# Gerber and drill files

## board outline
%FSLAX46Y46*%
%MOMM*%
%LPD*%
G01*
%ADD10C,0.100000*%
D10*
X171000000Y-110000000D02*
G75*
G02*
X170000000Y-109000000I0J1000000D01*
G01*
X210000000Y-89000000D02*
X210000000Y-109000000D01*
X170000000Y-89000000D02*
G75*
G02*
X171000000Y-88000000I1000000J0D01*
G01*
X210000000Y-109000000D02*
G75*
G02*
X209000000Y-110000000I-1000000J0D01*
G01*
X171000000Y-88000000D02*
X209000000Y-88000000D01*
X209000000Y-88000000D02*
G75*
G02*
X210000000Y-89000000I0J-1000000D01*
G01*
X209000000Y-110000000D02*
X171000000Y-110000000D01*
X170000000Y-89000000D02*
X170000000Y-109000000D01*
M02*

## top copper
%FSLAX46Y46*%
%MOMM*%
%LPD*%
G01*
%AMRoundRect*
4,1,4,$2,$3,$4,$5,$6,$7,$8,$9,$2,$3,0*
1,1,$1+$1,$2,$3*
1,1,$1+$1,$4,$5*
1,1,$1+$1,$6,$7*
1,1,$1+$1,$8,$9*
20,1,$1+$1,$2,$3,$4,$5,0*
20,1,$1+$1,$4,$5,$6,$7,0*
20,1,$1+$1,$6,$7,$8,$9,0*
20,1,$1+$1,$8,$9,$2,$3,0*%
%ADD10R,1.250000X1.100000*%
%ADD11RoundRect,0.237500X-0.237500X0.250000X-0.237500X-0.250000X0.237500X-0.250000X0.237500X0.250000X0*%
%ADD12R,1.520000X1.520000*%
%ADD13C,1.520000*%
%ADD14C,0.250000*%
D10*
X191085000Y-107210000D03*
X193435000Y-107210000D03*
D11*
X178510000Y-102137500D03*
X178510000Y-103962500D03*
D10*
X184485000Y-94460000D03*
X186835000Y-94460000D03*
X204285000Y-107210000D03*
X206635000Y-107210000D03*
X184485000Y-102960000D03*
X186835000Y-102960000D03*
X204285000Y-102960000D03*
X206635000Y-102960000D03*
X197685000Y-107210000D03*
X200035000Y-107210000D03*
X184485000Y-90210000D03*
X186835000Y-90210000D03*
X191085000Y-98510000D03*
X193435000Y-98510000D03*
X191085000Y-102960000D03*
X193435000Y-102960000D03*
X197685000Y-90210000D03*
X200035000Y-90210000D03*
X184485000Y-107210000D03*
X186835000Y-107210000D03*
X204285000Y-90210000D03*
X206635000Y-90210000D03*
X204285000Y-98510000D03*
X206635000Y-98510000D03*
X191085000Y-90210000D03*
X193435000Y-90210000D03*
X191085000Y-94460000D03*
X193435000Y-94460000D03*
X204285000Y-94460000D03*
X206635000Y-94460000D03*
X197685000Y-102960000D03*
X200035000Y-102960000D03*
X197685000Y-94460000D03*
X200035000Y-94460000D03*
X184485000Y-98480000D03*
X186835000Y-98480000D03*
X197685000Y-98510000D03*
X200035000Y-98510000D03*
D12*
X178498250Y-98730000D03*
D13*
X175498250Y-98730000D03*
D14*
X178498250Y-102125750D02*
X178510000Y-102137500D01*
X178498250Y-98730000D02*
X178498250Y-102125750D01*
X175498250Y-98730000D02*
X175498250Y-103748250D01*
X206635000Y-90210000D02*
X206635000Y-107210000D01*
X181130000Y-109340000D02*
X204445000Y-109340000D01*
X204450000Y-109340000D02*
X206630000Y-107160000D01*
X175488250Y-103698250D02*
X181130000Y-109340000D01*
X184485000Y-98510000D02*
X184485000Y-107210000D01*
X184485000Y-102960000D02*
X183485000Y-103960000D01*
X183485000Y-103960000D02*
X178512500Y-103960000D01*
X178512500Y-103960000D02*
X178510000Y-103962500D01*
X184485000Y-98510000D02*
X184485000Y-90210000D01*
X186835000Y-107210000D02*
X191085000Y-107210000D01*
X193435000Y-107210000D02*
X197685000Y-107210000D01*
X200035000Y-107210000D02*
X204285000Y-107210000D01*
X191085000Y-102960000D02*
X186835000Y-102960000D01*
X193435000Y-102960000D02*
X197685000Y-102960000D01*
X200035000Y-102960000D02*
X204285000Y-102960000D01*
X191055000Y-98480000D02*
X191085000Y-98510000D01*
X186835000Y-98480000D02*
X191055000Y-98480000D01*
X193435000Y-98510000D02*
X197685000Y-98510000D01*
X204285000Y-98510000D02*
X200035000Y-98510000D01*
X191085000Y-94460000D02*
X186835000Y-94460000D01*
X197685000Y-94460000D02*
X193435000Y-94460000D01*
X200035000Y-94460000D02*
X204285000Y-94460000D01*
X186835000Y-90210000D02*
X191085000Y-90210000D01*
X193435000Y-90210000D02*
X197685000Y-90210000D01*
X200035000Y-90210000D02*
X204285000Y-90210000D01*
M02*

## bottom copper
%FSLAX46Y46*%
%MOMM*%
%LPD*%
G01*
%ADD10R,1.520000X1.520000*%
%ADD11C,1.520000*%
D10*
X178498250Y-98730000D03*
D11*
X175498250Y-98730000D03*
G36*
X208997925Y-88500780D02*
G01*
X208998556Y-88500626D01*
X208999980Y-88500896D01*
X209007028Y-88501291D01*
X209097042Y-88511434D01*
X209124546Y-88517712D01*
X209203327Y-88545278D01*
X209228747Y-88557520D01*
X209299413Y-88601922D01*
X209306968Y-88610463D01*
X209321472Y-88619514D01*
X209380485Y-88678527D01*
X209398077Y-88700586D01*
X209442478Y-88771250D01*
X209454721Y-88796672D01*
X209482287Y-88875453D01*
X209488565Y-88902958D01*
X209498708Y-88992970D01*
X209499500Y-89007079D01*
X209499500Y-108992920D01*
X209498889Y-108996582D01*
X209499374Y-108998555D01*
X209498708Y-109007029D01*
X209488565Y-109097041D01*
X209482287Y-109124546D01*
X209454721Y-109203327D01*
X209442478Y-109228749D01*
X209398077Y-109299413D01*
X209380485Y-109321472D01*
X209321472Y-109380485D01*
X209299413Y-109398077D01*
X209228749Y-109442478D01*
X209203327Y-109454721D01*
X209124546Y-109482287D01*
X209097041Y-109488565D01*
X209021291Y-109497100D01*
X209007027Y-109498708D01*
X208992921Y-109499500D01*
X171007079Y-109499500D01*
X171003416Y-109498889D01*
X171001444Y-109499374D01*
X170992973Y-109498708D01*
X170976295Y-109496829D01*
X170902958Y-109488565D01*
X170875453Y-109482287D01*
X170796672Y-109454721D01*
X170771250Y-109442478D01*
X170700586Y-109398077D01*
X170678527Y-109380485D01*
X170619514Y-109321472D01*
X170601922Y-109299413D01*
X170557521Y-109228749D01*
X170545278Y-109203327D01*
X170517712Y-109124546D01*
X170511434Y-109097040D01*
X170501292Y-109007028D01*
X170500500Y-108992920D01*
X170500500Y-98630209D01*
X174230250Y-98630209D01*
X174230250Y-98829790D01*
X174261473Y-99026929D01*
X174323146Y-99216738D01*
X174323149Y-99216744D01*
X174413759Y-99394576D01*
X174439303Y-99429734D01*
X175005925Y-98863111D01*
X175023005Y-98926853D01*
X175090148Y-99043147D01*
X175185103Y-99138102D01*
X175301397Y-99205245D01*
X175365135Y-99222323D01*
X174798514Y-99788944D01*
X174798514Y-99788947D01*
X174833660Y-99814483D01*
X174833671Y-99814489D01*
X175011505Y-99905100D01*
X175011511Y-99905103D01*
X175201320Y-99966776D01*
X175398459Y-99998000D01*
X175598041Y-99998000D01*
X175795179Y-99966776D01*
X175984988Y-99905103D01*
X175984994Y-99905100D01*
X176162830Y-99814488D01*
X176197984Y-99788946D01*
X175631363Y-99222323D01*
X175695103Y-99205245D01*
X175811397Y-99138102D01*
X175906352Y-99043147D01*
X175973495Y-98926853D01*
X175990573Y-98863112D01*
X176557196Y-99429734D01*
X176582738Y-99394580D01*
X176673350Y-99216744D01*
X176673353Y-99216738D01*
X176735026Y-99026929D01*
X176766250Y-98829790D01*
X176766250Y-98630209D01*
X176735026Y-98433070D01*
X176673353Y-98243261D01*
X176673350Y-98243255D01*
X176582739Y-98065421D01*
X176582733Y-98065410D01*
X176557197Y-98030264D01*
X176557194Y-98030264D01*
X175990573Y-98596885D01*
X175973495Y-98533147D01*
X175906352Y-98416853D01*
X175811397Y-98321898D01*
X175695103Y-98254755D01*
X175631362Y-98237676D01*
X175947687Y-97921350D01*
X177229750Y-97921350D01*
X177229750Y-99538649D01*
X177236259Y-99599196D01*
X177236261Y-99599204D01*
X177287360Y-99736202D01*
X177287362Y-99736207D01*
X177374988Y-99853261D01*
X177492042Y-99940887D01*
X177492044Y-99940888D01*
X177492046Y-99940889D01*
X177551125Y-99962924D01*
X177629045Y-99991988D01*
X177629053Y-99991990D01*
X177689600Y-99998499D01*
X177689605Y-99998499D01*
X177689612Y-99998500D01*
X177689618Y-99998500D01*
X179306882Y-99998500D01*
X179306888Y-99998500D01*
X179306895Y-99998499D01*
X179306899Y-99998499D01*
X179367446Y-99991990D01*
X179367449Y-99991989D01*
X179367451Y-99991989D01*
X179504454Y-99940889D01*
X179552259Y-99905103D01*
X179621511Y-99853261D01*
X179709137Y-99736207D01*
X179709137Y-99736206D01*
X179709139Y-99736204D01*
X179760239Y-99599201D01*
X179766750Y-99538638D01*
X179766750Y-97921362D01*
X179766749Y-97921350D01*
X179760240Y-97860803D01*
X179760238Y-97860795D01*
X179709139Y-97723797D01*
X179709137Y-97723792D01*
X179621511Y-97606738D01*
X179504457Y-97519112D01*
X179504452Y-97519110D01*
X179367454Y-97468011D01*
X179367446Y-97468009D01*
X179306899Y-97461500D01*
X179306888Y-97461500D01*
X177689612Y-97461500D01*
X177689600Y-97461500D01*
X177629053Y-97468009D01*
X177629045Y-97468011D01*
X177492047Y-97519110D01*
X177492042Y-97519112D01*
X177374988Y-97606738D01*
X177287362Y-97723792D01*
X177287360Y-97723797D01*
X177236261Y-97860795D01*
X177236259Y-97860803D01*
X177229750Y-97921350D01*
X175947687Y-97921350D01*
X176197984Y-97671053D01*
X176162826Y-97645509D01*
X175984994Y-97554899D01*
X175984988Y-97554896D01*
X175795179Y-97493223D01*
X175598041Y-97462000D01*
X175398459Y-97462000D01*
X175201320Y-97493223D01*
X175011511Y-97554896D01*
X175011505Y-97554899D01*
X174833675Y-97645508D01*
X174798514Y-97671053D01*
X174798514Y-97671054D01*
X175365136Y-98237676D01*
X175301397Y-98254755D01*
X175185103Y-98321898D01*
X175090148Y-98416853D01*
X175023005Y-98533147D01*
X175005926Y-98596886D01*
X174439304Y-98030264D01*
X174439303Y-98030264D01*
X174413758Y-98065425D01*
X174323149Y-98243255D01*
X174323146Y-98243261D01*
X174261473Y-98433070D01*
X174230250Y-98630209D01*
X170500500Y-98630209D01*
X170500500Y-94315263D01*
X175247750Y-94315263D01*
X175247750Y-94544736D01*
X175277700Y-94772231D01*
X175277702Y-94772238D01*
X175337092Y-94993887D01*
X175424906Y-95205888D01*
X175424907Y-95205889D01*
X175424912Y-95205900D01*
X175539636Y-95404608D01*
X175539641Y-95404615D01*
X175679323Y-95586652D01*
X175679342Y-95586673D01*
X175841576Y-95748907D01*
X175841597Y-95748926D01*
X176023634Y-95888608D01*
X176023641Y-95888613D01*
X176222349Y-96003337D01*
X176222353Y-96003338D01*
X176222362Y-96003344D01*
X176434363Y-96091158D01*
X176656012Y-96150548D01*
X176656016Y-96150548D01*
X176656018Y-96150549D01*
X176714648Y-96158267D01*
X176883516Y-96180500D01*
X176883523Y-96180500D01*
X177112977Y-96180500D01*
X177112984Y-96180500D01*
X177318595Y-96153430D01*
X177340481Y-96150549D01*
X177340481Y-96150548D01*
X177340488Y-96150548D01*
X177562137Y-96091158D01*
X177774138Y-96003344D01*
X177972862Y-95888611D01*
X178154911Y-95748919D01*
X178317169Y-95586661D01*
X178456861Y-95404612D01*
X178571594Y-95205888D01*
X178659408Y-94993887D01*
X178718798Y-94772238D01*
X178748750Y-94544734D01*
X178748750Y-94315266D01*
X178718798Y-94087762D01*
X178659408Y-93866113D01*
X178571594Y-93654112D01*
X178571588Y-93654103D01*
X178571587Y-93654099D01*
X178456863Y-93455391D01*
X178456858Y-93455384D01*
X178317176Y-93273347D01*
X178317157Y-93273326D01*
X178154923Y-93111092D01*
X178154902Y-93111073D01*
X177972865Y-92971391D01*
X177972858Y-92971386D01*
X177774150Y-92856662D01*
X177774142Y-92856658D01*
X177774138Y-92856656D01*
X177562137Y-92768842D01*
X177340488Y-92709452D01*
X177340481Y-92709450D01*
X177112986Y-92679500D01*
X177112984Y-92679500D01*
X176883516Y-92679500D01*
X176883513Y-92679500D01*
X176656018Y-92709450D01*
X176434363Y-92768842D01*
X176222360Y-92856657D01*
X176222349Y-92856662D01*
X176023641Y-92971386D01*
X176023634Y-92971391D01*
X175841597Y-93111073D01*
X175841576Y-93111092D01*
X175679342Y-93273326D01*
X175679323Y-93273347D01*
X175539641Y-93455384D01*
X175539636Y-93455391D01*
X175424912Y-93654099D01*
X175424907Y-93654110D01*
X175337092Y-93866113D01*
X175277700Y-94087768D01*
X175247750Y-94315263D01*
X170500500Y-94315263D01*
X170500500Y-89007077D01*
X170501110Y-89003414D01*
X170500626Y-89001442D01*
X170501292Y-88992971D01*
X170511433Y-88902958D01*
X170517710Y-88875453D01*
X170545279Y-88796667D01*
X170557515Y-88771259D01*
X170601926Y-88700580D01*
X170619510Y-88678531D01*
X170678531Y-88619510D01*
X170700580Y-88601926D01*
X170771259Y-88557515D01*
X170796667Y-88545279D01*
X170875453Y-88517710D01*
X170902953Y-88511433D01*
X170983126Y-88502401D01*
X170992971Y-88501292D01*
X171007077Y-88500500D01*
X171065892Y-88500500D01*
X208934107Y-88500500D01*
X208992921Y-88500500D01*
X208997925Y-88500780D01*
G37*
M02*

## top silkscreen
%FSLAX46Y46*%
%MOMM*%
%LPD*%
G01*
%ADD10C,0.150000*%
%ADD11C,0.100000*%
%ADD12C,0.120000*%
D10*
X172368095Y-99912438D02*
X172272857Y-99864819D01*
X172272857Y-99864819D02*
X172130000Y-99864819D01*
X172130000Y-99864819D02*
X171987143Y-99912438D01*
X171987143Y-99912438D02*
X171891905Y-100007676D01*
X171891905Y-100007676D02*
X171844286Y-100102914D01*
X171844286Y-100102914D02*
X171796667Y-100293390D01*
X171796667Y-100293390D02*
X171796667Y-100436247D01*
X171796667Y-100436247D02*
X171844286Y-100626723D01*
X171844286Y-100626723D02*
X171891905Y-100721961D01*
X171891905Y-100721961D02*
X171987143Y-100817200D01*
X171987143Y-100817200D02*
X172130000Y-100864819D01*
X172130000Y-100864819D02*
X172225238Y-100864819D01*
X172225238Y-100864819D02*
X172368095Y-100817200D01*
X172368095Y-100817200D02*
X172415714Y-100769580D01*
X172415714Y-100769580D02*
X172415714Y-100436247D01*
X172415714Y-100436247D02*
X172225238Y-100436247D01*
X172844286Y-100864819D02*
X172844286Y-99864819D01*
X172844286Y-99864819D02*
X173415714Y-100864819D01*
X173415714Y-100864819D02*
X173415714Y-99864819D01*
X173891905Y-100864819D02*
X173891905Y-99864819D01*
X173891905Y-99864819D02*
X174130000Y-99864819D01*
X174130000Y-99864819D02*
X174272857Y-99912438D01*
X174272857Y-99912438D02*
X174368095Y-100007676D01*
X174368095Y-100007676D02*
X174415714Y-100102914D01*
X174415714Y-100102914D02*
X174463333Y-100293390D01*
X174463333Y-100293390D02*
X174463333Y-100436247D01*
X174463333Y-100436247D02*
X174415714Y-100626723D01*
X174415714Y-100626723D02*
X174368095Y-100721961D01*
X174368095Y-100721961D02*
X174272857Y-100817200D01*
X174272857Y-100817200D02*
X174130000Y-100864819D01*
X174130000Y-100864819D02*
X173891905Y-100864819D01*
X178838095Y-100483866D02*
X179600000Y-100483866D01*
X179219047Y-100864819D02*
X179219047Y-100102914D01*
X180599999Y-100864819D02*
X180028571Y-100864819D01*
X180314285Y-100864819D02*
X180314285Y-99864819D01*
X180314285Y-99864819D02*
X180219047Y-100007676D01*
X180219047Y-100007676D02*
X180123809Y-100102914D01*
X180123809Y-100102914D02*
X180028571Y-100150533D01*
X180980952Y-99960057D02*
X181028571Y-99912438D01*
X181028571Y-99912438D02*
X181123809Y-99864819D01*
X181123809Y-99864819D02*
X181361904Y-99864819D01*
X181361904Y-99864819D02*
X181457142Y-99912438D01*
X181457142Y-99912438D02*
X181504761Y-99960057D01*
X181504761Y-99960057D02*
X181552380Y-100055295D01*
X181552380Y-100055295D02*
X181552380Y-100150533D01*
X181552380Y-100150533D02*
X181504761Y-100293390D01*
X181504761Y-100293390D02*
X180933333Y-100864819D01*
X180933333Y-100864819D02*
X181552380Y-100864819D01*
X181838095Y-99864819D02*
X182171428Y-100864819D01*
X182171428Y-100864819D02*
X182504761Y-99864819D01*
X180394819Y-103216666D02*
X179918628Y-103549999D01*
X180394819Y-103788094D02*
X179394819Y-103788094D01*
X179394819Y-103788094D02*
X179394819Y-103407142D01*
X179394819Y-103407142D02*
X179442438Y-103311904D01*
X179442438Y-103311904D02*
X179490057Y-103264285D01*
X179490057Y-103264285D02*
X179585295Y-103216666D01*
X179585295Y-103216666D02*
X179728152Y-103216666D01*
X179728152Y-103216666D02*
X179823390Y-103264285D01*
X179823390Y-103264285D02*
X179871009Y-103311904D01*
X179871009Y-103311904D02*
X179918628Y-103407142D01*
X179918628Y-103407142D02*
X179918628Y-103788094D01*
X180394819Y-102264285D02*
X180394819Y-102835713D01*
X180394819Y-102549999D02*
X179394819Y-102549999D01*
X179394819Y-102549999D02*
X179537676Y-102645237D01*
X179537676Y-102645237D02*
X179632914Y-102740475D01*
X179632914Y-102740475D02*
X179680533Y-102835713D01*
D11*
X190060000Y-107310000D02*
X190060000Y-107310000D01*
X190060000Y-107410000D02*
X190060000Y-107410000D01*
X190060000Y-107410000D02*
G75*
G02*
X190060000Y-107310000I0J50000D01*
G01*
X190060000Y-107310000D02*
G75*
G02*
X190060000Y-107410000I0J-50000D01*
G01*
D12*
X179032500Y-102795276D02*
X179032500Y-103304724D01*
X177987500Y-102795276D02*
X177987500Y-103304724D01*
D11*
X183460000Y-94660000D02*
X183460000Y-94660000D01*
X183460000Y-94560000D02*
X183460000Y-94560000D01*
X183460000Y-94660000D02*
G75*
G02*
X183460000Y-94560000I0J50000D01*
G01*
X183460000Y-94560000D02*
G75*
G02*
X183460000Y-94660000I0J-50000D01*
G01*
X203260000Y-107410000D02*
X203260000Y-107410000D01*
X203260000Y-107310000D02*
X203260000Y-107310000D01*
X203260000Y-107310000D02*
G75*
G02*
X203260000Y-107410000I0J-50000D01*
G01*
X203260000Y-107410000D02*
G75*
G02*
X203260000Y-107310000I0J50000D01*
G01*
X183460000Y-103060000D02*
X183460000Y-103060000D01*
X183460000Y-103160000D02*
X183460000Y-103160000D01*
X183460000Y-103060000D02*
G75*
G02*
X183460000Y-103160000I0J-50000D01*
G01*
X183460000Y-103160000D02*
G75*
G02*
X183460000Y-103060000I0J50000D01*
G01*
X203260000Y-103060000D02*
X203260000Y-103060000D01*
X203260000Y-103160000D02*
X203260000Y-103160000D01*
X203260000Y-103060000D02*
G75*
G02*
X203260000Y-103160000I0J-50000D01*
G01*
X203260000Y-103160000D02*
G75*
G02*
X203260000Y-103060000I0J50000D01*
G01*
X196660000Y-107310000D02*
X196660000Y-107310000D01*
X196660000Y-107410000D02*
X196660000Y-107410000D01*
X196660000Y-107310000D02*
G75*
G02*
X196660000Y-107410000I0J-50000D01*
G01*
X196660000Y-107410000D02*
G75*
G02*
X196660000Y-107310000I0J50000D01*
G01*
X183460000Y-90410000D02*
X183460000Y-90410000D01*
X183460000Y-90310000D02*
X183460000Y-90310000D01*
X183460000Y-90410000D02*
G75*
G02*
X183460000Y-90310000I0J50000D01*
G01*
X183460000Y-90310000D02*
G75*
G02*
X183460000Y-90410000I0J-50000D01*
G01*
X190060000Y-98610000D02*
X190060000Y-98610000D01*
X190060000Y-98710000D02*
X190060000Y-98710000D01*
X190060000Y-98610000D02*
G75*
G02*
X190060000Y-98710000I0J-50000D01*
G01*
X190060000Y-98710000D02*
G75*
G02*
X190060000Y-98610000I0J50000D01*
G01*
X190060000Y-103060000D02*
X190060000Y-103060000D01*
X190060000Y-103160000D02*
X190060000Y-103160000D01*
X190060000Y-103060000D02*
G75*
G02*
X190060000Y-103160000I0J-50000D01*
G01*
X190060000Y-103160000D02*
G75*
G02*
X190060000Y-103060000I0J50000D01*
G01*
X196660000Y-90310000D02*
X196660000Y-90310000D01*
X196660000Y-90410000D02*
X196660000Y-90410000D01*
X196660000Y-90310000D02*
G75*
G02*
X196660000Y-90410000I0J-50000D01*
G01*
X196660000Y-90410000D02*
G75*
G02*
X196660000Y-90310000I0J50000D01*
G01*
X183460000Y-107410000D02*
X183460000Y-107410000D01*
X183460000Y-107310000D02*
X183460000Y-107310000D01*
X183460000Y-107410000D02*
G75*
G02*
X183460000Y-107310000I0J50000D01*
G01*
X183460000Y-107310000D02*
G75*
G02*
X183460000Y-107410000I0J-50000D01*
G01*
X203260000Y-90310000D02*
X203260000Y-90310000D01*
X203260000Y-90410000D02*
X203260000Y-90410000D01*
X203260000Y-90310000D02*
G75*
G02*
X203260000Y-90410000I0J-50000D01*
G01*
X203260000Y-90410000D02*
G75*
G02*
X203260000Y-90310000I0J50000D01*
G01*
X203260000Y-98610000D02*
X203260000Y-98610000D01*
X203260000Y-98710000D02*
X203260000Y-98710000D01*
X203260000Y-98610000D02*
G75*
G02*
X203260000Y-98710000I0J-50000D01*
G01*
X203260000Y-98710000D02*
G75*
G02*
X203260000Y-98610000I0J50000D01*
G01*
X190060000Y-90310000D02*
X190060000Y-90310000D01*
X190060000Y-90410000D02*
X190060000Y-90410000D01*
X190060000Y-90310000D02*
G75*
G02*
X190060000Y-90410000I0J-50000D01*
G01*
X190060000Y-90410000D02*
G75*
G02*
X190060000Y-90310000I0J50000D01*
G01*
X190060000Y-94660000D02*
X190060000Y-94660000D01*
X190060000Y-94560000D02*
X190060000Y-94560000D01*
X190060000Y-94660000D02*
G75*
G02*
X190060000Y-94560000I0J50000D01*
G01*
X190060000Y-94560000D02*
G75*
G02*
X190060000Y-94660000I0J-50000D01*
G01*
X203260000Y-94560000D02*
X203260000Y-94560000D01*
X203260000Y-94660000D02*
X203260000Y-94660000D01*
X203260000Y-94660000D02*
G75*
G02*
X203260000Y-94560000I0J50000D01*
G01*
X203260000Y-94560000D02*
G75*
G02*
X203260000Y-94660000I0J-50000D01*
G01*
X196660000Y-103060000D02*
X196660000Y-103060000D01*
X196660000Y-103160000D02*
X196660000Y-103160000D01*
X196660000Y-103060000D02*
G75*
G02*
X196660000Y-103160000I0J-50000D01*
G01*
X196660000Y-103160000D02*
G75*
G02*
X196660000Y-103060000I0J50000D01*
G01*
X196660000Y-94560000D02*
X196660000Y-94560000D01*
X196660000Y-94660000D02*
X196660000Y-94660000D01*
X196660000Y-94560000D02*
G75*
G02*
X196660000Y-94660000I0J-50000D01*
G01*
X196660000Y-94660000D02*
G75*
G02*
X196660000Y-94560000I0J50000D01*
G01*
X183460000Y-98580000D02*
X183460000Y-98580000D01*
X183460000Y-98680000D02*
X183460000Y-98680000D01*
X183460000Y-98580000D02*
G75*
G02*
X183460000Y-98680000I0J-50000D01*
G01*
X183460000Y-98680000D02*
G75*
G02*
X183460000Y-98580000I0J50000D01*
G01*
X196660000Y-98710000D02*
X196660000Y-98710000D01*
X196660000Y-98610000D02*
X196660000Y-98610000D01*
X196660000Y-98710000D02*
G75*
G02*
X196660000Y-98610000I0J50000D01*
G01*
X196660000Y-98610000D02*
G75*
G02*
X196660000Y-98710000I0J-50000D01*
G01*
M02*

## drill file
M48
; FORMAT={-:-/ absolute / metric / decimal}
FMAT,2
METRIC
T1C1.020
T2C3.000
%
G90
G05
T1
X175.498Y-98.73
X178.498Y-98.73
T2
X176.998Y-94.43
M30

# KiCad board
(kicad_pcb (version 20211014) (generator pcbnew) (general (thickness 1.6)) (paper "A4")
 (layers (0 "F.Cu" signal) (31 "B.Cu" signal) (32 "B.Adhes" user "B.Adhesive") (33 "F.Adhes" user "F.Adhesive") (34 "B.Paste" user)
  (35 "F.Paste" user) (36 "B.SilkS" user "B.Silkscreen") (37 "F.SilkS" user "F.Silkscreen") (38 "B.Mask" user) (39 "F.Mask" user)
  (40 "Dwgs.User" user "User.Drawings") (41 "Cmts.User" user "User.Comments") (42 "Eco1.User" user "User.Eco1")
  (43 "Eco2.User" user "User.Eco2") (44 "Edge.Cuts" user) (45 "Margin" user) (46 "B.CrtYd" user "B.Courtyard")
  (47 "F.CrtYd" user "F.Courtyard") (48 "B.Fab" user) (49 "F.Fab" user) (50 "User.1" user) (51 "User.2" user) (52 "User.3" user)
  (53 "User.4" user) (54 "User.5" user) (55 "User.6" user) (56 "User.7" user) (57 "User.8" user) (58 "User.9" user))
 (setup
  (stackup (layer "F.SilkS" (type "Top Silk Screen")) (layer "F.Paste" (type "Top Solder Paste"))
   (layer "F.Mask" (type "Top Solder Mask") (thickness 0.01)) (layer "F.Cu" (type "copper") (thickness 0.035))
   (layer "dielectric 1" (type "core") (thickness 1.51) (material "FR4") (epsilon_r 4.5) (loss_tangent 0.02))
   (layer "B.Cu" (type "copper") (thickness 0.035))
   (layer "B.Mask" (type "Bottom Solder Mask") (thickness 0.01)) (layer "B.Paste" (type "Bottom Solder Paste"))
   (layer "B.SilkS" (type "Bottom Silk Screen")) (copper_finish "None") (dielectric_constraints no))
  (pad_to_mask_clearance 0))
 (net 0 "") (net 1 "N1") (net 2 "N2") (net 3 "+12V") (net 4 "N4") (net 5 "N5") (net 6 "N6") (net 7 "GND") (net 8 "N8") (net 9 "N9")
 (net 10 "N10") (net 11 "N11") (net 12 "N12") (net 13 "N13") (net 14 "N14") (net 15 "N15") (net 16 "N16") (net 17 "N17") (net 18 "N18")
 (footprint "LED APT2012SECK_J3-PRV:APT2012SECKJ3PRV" (layer "F.Cu") (at 192.26 107.21)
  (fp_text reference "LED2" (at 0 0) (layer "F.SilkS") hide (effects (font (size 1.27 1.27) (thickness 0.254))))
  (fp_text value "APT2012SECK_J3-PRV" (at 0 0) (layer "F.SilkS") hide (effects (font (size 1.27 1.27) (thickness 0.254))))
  (fp_line (start -2.2 0.1) (end -2.2 0.1) (layer "F.SilkS") (width 0.1))
  (fp_line (start -2.2 0.2) (end -2.2 0.2) (layer "F.SilkS") (width 0.1))
  (fp_arc (start -2.2 0.2) (mid -2.25 0.15) (end -2.2 0.1) (layer "F.SilkS") (width 0.1))
  (fp_arc (start -2.2 0.1) (mid -2.15 0.15) (end -2.2 0.2) (layer "F.SilkS") (width 0.1))
  (pad "1" smd rect (at -1.175 0 90) (size 1.1 1.25) (layers "F.Cu" "F.Paste" "F.Mask") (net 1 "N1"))
  (pad "2" smd rect (at 1.175 0 90) (size 1.1 1.25) (layers "F.Cu" "F.Paste" "F.Mask") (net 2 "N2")))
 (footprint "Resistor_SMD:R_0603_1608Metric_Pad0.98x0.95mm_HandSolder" (layer "F.Cu") (at 178.51 103.05 -90)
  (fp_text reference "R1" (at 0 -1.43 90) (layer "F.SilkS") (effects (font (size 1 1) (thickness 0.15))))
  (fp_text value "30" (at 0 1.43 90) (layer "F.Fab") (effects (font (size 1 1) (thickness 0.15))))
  (fp_line (start -0.254724 -0.5225) (end 0.254724 -0.5225) (layer "F.SilkS") (width 0.12))
  (fp_line (start -0.254724 0.5225) (end 0.254724 0.5225) (layer "F.SilkS") (width 0.12))
  (pad "1" smd roundrect locked (at -0.9125 0 270) (size 0.975 0.95) (layers "F.Cu" "F.Paste" "F.Mask") (roundrect_rratio 0.25)
   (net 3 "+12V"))
  (pad "2" smd roundrect locked (at 0.9125 0 270) (size 0.975 0.95) (layers "F.Cu" "F.Paste" "F.Mask") (roundrect_rratio 0.25) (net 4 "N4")))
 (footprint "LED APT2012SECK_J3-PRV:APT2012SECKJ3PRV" (layer "F.Cu") (at 185.66 94.46)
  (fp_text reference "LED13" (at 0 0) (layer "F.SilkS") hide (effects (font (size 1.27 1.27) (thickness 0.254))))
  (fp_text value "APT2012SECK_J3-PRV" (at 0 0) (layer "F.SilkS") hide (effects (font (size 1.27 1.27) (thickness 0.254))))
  (fp_line (start -2.2 0.2) (end -2.2 0.2) (layer "F.SilkS") (width 0.1))
  (fp_line (start -2.2 0.1) (end -2.2 0.1) (layer "F.SilkS") (width 0.1))
  (fp_arc (start -2.2 0.2) (mid -2.25 0.15) (end -2.2 0.1) (layer "F.SilkS") (width 0.1))
  (fp_arc (start -2.2 0.1) (mid -2.15 0.15) (end -2.2 0.2) (layer "F.SilkS") (width 0.1))
  (pad "1" smd rect (at -1.175 0 90) (size 1.1 1.25) (layers "F.Cu" "F.Paste" "F.Mask") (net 4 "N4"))
  (pad "2" smd rect (at 1.175 0 90) (size 1.1 1.25) (layers "F.Cu" "F.Paste" "F.Mask") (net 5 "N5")))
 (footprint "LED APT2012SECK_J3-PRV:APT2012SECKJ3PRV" (layer "F.Cu") (at 205.46 107.21)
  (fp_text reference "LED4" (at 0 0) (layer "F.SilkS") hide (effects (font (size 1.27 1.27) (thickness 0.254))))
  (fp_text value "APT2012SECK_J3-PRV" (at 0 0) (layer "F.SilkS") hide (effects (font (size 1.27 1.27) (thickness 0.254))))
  (fp_line (start -2.2 0.2) (end -2.2 0.2) (layer "F.SilkS") (width 0.1))
  (fp_line (start -2.2 0.1) (end -2.2 0.1) (layer "F.SilkS") (width 0.1))
  (fp_arc (start -2.2 0.1) (mid -2.15 0.15) (end -2.2 0.2) (layer "F.SilkS") (width 0.1))
  (fp_arc (start -2.2 0.2) (mid -2.25 0.15) (end -2.2 0.1) (layer "F.SilkS") (width 0.1))
  (pad "1" smd rect (at -1.175 0 90) (size 1.1 1.25) (layers "F.Cu" "F.Paste" "F.Mask") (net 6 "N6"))
  (pad "2" smd rect (at 1.175 0 90) (size 1.1 1.25) (layers "F.Cu" "F.Paste" "F.Mask") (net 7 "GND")))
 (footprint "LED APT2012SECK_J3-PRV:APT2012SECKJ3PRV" (layer "F.Cu") (at 185.66 102.96)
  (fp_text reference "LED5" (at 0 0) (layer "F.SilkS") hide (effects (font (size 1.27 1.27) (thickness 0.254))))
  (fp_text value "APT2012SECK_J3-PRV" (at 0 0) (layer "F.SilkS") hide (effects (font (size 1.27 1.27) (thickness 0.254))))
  (fp_line (start -2.2 0.1) (end -2.2 0.1) (layer "F.SilkS") (width 0.1))
  (fp_line (start -2.2 0.2) (end -2.2 0.2) (layer "F.SilkS") (width 0.1))
  (fp_arc (start -2.2 0.1) (mid -2.15 0.15) (end -2.2 0.2) (layer "F.SilkS") (width 0.1))
  (fp_arc (start -2.2 0.2) (mid -2.25 0.15) (end -2.2 0.1) (layer "F.SilkS") (width 0.1))
  (pad "1" smd rect (at -1.175 0 90) (size 1.1 1.25) (layers "F.Cu" "F.Paste" "F.Mask") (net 4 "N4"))
  (pad "2" smd rect (at 1.175 0 90) (size 1.1 1.25) (layers "F.Cu" "F.Paste" "F.Mask") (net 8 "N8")))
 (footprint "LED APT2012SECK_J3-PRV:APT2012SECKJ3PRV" (layer "F.Cu") (at 205.46 102.96)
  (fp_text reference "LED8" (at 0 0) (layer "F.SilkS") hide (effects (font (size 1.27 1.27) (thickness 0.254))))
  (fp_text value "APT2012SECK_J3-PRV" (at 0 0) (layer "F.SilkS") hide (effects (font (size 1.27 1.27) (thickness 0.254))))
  (fp_line (start -2.2 0.1) (end -2.2 0.1) (layer "F.SilkS") (width 0.1))
  (fp_line (start -2.2 0.2) (end -2.2 0.2) (layer "F.SilkS") (width 0.1))
  (fp_arc (start -2.2 0.1) (mid -2.15 0.15) (end -2.2 0.2) (layer "F.SilkS") (width 0.1))
  (fp_arc (start -2.2 0.2) (mid -2.25 0.15) (end -2.2 0.1) (layer "F.SilkS") (width 0.1))
  (pad "1" smd rect (at -1.175 0 90) (size 1.1 1.25) (layers "F.Cu" "F.Paste" "F.Mask") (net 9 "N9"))
  (pad "2" smd rect (at 1.175 0 90) (size 1.1 1.25) (layers "F.Cu" "F.Paste" "F.Mask") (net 7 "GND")))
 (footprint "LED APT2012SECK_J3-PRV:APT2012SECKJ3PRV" (layer "F.Cu") (at 198.86 107.21)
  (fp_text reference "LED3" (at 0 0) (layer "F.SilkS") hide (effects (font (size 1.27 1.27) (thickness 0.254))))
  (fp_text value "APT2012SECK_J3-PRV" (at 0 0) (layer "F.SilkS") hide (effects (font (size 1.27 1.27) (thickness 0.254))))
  (fp_line (start -2.2 0.1) (end -2.2 0.1) (layer "F.SilkS") (width 0.1))
  (fp_line (start -2.2 0.2) (end -2.2 0.2) (layer "F.SilkS") (width 0.1))
  (fp_arc (start -2.2 0.1) (mid -2.15 0.15) (end -2.2 0.2) (layer "F.SilkS") (width 0.1))
  (fp_arc (start -2.2 0.2) (mid -2.25 0.15) (end -2.2 0.1) (layer "F.SilkS") (width 0.1))
  (pad "1" smd rect (at -1.175 0 90) (size 1.1 1.25) (layers "F.Cu" "F.Paste" "F.Mask") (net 2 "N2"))
  (pad "2" smd rect (at 1.175 0 90) (size 1.1 1.25) (layers "F.Cu" "F.Paste" "F.Mask") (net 6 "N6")))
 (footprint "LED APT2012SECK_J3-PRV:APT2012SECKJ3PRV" (layer "F.Cu") (at 185.66 90.21)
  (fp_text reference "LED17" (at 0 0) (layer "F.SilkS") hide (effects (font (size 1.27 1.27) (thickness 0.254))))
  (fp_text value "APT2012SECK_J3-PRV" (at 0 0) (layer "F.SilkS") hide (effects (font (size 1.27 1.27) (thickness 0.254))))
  (fp_line (start -2.2 0.2) (end -2.2 0.2) (layer "F.SilkS") (width 0.1))
  (fp_line (start -2.2 0.1) (end -2.2 0.1) (layer "F.SilkS") (width 0.1))
  (fp_arc (start -2.2 0.2) (mid -2.25 0.15) (end -2.2 0.1) (layer "F.SilkS") (width 0.1))
  (fp_arc (start -2.2 0.1) (mid -2.15 0.15) (end -2.2 0.2) (layer "F.SilkS") (width 0.1))
  (pad "1" smd rect (at -1.175 0 90) (size 1.1 1.25) (layers "F.Cu" "F.Paste" "F.Mask") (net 4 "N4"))
  (pad "2" smd rect (at 1.175 0 90) (size 1.1 1.25) (layers "F.Cu" "F.Paste" "F.Mask") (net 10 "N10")))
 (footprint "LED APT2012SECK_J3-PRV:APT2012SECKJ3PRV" (layer "F.Cu") (at 192.26 98.51)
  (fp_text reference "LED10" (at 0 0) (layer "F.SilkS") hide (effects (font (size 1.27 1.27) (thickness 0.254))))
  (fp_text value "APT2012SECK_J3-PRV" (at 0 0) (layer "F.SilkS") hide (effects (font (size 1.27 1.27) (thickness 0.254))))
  (fp_line (start -2.2 0.1) (end -2.2 0.1) (layer "F.SilkS") (width 0.1))
  (fp_line (start -2.2 0.2) (end -2.2 0.2) (layer "F.SilkS") (width 0.1))
  (fp_arc (start -2.2 0.1) (mid -2.15 0.15) (end -2.2 0.2) (layer "F.SilkS") (width 0.1))
  (fp_arc (start -2.2 0.2) (mid -2.25 0.15) (end -2.2 0.1) (layer "F.SilkS") (width 0.1))
  (pad "1" smd rect (at -1.175 0 90) (size 1.1 1.25) (layers "F.Cu" "F.Paste" "F.Mask") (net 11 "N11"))
  (pad "2" smd rect (at 1.175 0 90) (size 1.1 1.25) (layers "F.Cu" "F.Paste" "F.Mask") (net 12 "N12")))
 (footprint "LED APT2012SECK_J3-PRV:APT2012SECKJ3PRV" (layer "F.Cu") (at 192.26 102.96)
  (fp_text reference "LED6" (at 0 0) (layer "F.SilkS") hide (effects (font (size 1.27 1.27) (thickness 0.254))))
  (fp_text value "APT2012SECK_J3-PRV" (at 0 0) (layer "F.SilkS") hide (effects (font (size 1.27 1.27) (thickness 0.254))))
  (fp_line (start -2.2 0.1) (end -2.2 0.1) (layer "F.SilkS") (width 0.1))
  (fp_line (start -2.2 0.2) (end -2.2 0.2) (layer "F.SilkS") (width 0.1))
  (fp_arc (start -2.2 0.1) (mid -2.15 0.15) (end -2.2 0.2) (layer "F.SilkS") (width 0.1))
  (fp_arc (start -2.2 0.2) (mid -2.25 0.15) (end -2.2 0.1) (layer "F.SilkS") (width 0.1))
  (pad "1" smd rect (at -1.175 0 90) (size 1.1 1.25) (layers "F.Cu" "F.Paste" "F.Mask") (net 8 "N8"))
  (pad "2" smd rect (at 1.175 0 90) (size 1.1 1.25) (layers "F.Cu" "F.Paste" "F.Mask") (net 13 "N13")))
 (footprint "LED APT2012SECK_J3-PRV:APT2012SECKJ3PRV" (layer "F.Cu") (at 198.86 90.21)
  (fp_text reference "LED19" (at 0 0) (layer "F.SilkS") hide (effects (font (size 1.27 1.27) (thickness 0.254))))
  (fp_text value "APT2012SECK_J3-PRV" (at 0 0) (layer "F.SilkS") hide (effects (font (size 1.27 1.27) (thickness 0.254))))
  (fp_line (start -2.2 0.1) (end -2.2 0.1) (layer "F.SilkS") (width 0.1))
  (fp_line (start -2.2 0.2) (end -2.2 0.2) (layer "F.SilkS") (width 0.1))
  (fp_arc (start -2.2 0.1) (mid -2.15 0.15) (end -2.2 0.2) (layer "F.SilkS") (width 0.1))
  (fp_arc (start -2.2 0.2) (mid -2.25 0.15) (end -2.2 0.1) (layer "F.SilkS") (width 0.1))
  (pad "1" smd rect (at -1.175 0 90) (size 1.1 1.25) (layers "F.Cu" "F.Paste" "F.Mask") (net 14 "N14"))
  (pad "2" smd rect (at 1.175 0 90) (size 1.1 1.25) (layers "F.Cu" "F.Paste" "F.Mask") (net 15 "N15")))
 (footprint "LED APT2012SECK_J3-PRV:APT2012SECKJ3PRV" (layer "F.Cu") (at 185.66 107.21)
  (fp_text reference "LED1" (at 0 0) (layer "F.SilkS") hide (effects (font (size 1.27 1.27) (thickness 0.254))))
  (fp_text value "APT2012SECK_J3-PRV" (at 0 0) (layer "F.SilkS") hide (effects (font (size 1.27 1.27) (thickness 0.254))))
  (fp_line (start -2.2 0.2) (end -2.2 0.2) (layer "F.SilkS") (width 0.1))
  (fp_line (start -2.2 0.1) (end -2.2 0.1) (layer "F.SilkS") (width 0.1))
  (fp_arc (start -2.2 0.2) (mid -2.25 0.15) (end -2.2 0.1) (layer "F.SilkS") (width 0.1))
  (fp_arc (start -2.2 0.1) (mid -2.15 0.15) (end -2.2 0.2) (layer "F.SilkS") (width 0.1))
  (pad "1" smd rect (at -1.175 0 90) (size 1.1 1.25) (layers "F.Cu" "F.Paste" "F.Mask") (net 4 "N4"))
  (pad "2" smd rect (at 1.175 0 90) (size 1.1 1.25) (layers "F.Cu" "F.Paste" "F.Mask") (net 1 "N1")))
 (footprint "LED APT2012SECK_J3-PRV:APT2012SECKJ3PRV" (layer "F.Cu") (at 205.46 90.21)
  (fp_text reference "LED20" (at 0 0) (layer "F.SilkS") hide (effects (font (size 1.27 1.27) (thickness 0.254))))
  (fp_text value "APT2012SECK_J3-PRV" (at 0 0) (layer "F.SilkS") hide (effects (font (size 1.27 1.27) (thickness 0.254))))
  (fp_line (start -2.2 0.1) (end -2.2 0.1) (layer "F.SilkS") (width 0.1))
  (fp_line (start -2.2 0.2) (end -2.2 0.2) (layer "F.SilkS") (width 0.1))
  (fp_arc (start -2.2 0.1) (mid -2.15 0.15) (end -2.2 0.2) (layer "F.SilkS") (width 0.1))
  (fp_arc (start -2.2 0.2) (mid -2.25 0.15) (end -2.2 0.1) (layer "F.SilkS") (width 0.1))
  (pad "1" smd rect (at -1.175 0 90) (size 1.1 1.25) (layers "F.Cu" "F.Paste" "F.Mask") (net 15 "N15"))
  (pad "2" smd rect (at 1.175 0 90) (size 1.1 1.25) (layers "F.Cu" "F.Paste" "F.Mask") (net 7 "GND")))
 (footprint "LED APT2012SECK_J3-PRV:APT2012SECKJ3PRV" (layer "F.Cu") (at 205.46 98.51)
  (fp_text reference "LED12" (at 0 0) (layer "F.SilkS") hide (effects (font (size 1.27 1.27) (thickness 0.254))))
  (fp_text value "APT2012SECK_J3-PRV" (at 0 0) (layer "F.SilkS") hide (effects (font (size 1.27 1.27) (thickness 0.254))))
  (fp_line (start -2.2 0.1) (end -2.2 0.1) (layer "F.SilkS") (width 0.1))
  (fp_line (start -2.2 0.2) (end -2.2 0.2) (layer "F.SilkS") (width 0.1))
  (fp_arc (start -2.2 0.1) (mid -2.15 0.15) (end -2.2 0.2) (layer "F.SilkS") (width 0.1))
  (fp_arc (start -2.2 0.2) (mid -2.25 0.15) (end -2.2 0.1) (layer "F.SilkS") (width 0.1))
  (pad "1" smd rect (at -1.175 0 90) (size 1.1 1.25) (layers "F.Cu" "F.Paste" "F.Mask") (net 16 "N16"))
  (pad "2" smd rect (at 1.175 0 90) (size 1.1 1.25) (layers "F.Cu" "F.Paste" "F.Mask") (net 7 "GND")))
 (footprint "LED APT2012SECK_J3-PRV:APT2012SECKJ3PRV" (layer "F.Cu") (at 192.26 90.21)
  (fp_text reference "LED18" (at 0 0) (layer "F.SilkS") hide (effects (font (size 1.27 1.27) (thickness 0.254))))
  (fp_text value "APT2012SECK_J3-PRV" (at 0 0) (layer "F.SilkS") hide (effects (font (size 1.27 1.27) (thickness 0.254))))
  (fp_line (start -2.2 0.1) (end -2.2 0.1) (layer "F.SilkS") (width 0.1))
  (fp_line (start -2.2 0.2) (end -2.2 0.2) (layer "F.SilkS") (width 0.1))
  (fp_arc (start -2.2 0.1) (mid -2.15 0.15) (end -2.2 0.2) (layer "F.SilkS") (width 0.1))
  (fp_arc (start -2.2 0.2) (mid -2.25 0.15) (end -2.2 0.1) (layer "F.SilkS") (width 0.1))
  (pad "1" smd rect (at -1.175 0 90) (size 1.1 1.25) (layers "F.Cu" "F.Paste" "F.Mask") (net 10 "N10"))
  (pad "2" smd rect (at 1.175 0 90) (size 1.1 1.25) (layers "F.Cu" "F.Paste" "F.Mask") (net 14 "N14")))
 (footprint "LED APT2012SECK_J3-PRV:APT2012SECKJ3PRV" (layer "F.Cu") (at 192.26 94.46)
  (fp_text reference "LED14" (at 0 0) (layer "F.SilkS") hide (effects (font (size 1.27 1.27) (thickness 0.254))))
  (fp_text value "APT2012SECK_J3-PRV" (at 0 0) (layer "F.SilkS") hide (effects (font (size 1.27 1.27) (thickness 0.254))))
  (fp_line (start -2.2 0.2) (end -2.2 0.2) (layer "F.SilkS") (width 0.1))
  (fp_line (start -2.2 0.1) (end -2.2 0.1) (layer "F.SilkS") (width 0.1))
  (fp_arc (start -2.2 0.2) (mid -2.25 0.15) (end -2.2 0.1) (layer "F.SilkS") (width 0.1))
  (fp_arc (start -2.2 0.1) (mid -2.15 0.15) (end -2.2 0.2) (layer "F.SilkS") (width 0.1))
  (pad "1" smd rect (at -1.175 0 90) (size 1.1 1.25) (layers "F.Cu" "F.Paste" "F.Mask") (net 5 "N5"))
  (pad "2" smd rect (at 1.175 0 90) (size 1.1 1.25) (layers "F.Cu" "F.Paste" "F.Mask") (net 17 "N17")))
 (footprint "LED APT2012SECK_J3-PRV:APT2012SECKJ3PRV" (layer "F.Cu") (at 205.46 94.46)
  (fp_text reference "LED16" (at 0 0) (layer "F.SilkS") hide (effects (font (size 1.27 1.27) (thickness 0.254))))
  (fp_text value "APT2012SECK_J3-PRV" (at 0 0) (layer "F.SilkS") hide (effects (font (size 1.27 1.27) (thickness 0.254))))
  (fp_line (start -2.2 0.1) (end -2.2 0.1) (layer "F.SilkS") (width 0.1))
  (fp_line (start -2.2 0.2) (end -2.2 0.2) (layer "F.SilkS") (width 0.1))
  (fp_arc (start -2.2 0.2) (mid -2.25 0.15) (end -2.2 0.1) (layer "F.SilkS") (width 0.1))
  (fp_arc (start -2.2 0.1) (mid -2.15 0.15) (end -2.2 0.2) (layer "F.SilkS") (width 0.1))
  (pad "1" smd rect (at -1.175 0 90) (size 1.1 1.25) (layers "F.Cu" "F.Paste" "F.Mask") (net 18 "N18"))
  (pad "2" smd rect (at 1.175 0 90) (size 1.1 1.25) (layers "F.Cu" "F.Paste" "F.Mask") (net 7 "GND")))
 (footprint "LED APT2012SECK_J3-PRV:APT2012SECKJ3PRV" (layer "F.Cu") (at 198.86 102.96)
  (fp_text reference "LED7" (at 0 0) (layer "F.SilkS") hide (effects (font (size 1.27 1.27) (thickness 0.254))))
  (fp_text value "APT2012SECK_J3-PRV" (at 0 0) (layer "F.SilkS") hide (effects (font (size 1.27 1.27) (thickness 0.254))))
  (fp_line (start -2.2 0.1) (end -2.2 0.1) (layer "F.SilkS") (width 0.1))
  (fp_line (start -2.2 0.2) (end -2.2 0.2) (layer "F.SilkS") (width 0.1))
  (fp_arc (start -2.2 0.1) (mid -2.15 0.15) (end -2.2 0.2) (layer "F.SilkS") (width 0.1))
  (fp_arc (start -2.2 0.2) (mid -2.25 0.15) (end -2.2 0.1) (layer "F.SilkS") (width 0.1))
  (pad "1" smd rect (at -1.175 0 90) (size 1.1 1.25) (layers "F.Cu" "F.Paste" "F.Mask") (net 13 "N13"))
  (pad "2" smd rect (at 1.175 0 90) (size 1.1 1.25) (layers "F.Cu" "F.Paste" "F.Mask") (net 9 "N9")))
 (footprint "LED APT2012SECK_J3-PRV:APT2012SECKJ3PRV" (layer "F.Cu") (at 198.86 94.46)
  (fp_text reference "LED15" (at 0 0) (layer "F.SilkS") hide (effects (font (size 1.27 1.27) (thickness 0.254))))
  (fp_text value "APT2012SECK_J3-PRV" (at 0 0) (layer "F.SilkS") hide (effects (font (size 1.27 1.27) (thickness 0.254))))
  (fp_line (start -2.2 0.1) (end -2.2 0.1) (layer "F.SilkS") (width 0.1))
  (fp_line (start -2.2 0.2) (end -2.2 0.2) (layer "F.SilkS") (width 0.1))
  (fp_arc (start -2.2 0.1) (mid -2.15 0.15) (end -2.2 0.2) (layer "F.SilkS") (width 0.1))
  (fp_arc (start -2.2 0.2) (mid -2.25 0.15) (end -2.2 0.1) (layer "F.SilkS") (width 0.1))
  (pad "1" smd rect (at -1.175 0 90) (size 1.1 1.25) (layers "F.Cu" "F.Paste" "F.Mask") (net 17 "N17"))
  (pad "2" smd rect (at 1.175 0 90) (size 1.1 1.25) (layers "F.Cu" "F.Paste" "F.Mask") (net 18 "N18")))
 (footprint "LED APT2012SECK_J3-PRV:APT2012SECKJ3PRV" (layer "F.Cu") (at 185.66 98.48)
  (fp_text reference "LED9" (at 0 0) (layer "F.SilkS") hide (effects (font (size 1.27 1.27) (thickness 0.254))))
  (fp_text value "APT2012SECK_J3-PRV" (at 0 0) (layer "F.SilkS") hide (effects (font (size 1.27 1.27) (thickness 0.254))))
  (fp_line (start -2.2 0.1) (end -2.2 0.1) (layer "F.SilkS") (width 0.1))
  (fp_line (start -2.2 0.2) (end -2.2 0.2) (layer "F.SilkS") (width 0.1))
  (fp_arc (start -2.2 0.1) (mid -2.15 0.15) (end -2.2 0.2) (layer "F.SilkS") (width 0.1))
  (fp_arc (start -2.2 0.2) (mid -2.25 0.15) (end -2.2 0.1) (layer "F.SilkS") (width 0.1))
  (pad "1" smd rect (at -1.175 0 90) (size 1.1 1.25) (layers "F.Cu" "F.Paste" "F.Mask") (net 4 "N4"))
  (pad "2" smd rect (at 1.175 0 90) (size 1.1 1.25) (layers "F.Cu" "F.Paste" "F.Mask") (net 11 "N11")))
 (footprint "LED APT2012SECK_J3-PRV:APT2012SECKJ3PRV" (layer "F.Cu") (at 198.86 98.51)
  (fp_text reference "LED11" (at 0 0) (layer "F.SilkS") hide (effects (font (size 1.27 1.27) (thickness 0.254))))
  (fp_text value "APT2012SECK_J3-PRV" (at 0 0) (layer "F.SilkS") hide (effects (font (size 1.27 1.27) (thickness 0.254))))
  (fp_line (start -2.2 0.2) (end -2.2 0.2) (layer "F.SilkS") (width 0.1))
  (fp_line (start -2.2 0.1) (end -2.2 0.1) (layer "F.SilkS") (width 0.1))
  (fp_arc (start -2.2 0.2) (mid -2.25 0.15) (end -2.2 0.1) (layer "F.SilkS") (width 0.1))
  (fp_arc (start -2.2 0.1) (mid -2.15 0.15) (end -2.2 0.2) (layer "F.SilkS") (width 0.1))
  (pad "1" smd rect (at -1.175 0 90) (size 1.1 1.25) (layers "F.Cu" "F.Paste" "F.Mask") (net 12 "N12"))
  (pad "2" smd rect (at 1.175 0 90) (size 1.1 1.25) (layers "F.Cu" "F.Paste" "F.Mask") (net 16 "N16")))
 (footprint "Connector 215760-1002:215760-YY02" (layer "B.Cu") (at 178.49825 98.73)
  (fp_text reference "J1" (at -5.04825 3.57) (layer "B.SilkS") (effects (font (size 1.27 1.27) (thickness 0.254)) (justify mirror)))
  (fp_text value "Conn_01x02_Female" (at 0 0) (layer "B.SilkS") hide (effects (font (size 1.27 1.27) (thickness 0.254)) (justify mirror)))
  (pad "" np_thru_hole circle locked (at -1.5 -4.3) (size 3 3) (drill 3) (layers *.Cu *.Mask))
  (pad "1" thru_hole rect locked (at 0 0) (size 1.52 1.52) (drill 1.02) (layers *.Cu *.Mask) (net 3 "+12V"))
  (pad "2" thru_hole circle locked (at -3 0) (size 1.52 1.52) (drill 1.02) (layers *.Cu *.Mask) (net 7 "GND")))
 (gr_arc (start 171 110) (mid 170.292894 109.707107) (end 170 109) (layer "Edge.Cuts") (width 0.1))
 (gr_line (start 210 89) (end 210 109) (layer "Edge.Cuts") (width 0.1))
 (gr_arc (start 170 89) (mid 170.292893 88.292893) (end 171 88) (layer "Edge.Cuts") (width 0.1))
 (gr_arc (start 210 109) (mid 209.707107 109.707106) (end 209 110) (layer "Edge.Cuts") (width 0.1))
 (gr_line (start 171 88) (end 209 88) (layer "Edge.Cuts") (width 0.1))
 (gr_arc (start 209 88) (mid 209.707106 88.292893) (end 210 89) (layer "Edge.Cuts") (width 0.1))
 (gr_line (start 209 110) (end 171 110) (layer "Edge.Cuts") (width 0.1))
 (gr_line (start 170 89) (end 170 109) (layer "Edge.Cuts") (width 0.1))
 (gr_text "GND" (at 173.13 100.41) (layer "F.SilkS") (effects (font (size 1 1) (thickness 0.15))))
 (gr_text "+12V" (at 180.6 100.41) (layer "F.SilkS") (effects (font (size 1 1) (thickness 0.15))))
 (segment (start 178.49825 102.12575) (end 178.51 102.1375) (width 0.25) (layer "F.Cu") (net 3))
 (segment (start 178.49825 98.73) (end 178.49825 102.12575) (width 0.25) (layer "F.Cu") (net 3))
 (segment (start 175.49825 98.73) (end 175.49825 103.74825) (width 0.25) (layer "F.Cu") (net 7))
 (segment (start 206.635 90.21) (end 206.635 107.21) (width 0.25) (layer "F.Cu") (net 7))
 (segment (start 181.13 109.34) (end 204.445 109.34) (width 0.25) (layer "F.Cu") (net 7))
 (segment (start 204.45 109.34) (end 206.63 107.16) (width 0.25) (layer "F.Cu") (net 7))
 (segment (start 175.48825 103.69825) (end 181.13 109.34) (width 0.25) (layer "F.Cu") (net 7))
 (segment (start 184.485 98.51) (end 184.485 107.21) (width 0.25) (layer "F.Cu") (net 4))
 (segment (start 184.485 102.96) (end 183.485 103.96) (width 0.25) (layer "F.Cu") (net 4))
 (segment (start 183.485 103.96) (end 178.5125 103.96) (width 0.25) (layer "F.Cu") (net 4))
 (segment (start 178.5125 103.96) (end 178.51 103.9625) (width 0.25) (layer "F.Cu") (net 4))
 (segment (start 184.485 98.51) (end 184.485 90.21) (width 0.25) (layer "F.Cu") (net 4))
 (segment (start 186.835 107.21) (end 191.085 107.21) (width 0.25) (layer "F.Cu") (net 1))
 (segment (start 193.435 107.21) (end 197.685 107.21) (width 0.25) (layer "F.Cu") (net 2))
 (segment (start 200.035 107.21) (end 204.285 107.21) (width 0.25) (layer "F.Cu") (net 6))
 (segment (start 191.085 102.96) (end 186.835 102.96) (width 0.25) (layer "F.Cu") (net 8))
 (segment (start 193.435 102.96) (end 197.685 102.96) (width 0.25) (layer "F.Cu") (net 13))
 (segment (start 200.035 102.96) (end 204.285 102.96) (width 0.25) (layer "F.Cu") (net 9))
 (segment (start 191.055 98.48) (end 191.085 98.51) (width 0.25) (layer "F.Cu") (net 11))
 (segment (start 186.835 98.48) (end 191.055 98.48) (width 0.25) (layer "F.Cu") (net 11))
 (segment (start 193.435 98.51) (end 197.685 98.51) (width 0.25) (layer "F.Cu") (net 12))
 (segment (start 204.285 98.51) (end 200.035 98.51) (width 0.25) (layer "F.Cu") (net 16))
 (segment (start 191.085 94.46) (end 186.835 94.46) (width 0.25) (layer "F.Cu") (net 5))
 (segment (start 197.685 94.46) (end 193.435 94.46) (width 0.25) (layer "F.Cu") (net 17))
 (segment (start 200.035 94.46) (end 204.285 94.46) (width 0.25) (layer "F.Cu") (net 18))
 (segment (start 186.835 90.21) (end 191.085 90.21) (width 0.25) (layer "F.Cu") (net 10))
 (segment (start 193.435 90.21) (end 197.685 90.21) (width 0.25) (layer "F.Cu") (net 14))
 (segment (start 200.035 90.21) (end 204.285 90.21) (width 0.25) (layer "F.Cu") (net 15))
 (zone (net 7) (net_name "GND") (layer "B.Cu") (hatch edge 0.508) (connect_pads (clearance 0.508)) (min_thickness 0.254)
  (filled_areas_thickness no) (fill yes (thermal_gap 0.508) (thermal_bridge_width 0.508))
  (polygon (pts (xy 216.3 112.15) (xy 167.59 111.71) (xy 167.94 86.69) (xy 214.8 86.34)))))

